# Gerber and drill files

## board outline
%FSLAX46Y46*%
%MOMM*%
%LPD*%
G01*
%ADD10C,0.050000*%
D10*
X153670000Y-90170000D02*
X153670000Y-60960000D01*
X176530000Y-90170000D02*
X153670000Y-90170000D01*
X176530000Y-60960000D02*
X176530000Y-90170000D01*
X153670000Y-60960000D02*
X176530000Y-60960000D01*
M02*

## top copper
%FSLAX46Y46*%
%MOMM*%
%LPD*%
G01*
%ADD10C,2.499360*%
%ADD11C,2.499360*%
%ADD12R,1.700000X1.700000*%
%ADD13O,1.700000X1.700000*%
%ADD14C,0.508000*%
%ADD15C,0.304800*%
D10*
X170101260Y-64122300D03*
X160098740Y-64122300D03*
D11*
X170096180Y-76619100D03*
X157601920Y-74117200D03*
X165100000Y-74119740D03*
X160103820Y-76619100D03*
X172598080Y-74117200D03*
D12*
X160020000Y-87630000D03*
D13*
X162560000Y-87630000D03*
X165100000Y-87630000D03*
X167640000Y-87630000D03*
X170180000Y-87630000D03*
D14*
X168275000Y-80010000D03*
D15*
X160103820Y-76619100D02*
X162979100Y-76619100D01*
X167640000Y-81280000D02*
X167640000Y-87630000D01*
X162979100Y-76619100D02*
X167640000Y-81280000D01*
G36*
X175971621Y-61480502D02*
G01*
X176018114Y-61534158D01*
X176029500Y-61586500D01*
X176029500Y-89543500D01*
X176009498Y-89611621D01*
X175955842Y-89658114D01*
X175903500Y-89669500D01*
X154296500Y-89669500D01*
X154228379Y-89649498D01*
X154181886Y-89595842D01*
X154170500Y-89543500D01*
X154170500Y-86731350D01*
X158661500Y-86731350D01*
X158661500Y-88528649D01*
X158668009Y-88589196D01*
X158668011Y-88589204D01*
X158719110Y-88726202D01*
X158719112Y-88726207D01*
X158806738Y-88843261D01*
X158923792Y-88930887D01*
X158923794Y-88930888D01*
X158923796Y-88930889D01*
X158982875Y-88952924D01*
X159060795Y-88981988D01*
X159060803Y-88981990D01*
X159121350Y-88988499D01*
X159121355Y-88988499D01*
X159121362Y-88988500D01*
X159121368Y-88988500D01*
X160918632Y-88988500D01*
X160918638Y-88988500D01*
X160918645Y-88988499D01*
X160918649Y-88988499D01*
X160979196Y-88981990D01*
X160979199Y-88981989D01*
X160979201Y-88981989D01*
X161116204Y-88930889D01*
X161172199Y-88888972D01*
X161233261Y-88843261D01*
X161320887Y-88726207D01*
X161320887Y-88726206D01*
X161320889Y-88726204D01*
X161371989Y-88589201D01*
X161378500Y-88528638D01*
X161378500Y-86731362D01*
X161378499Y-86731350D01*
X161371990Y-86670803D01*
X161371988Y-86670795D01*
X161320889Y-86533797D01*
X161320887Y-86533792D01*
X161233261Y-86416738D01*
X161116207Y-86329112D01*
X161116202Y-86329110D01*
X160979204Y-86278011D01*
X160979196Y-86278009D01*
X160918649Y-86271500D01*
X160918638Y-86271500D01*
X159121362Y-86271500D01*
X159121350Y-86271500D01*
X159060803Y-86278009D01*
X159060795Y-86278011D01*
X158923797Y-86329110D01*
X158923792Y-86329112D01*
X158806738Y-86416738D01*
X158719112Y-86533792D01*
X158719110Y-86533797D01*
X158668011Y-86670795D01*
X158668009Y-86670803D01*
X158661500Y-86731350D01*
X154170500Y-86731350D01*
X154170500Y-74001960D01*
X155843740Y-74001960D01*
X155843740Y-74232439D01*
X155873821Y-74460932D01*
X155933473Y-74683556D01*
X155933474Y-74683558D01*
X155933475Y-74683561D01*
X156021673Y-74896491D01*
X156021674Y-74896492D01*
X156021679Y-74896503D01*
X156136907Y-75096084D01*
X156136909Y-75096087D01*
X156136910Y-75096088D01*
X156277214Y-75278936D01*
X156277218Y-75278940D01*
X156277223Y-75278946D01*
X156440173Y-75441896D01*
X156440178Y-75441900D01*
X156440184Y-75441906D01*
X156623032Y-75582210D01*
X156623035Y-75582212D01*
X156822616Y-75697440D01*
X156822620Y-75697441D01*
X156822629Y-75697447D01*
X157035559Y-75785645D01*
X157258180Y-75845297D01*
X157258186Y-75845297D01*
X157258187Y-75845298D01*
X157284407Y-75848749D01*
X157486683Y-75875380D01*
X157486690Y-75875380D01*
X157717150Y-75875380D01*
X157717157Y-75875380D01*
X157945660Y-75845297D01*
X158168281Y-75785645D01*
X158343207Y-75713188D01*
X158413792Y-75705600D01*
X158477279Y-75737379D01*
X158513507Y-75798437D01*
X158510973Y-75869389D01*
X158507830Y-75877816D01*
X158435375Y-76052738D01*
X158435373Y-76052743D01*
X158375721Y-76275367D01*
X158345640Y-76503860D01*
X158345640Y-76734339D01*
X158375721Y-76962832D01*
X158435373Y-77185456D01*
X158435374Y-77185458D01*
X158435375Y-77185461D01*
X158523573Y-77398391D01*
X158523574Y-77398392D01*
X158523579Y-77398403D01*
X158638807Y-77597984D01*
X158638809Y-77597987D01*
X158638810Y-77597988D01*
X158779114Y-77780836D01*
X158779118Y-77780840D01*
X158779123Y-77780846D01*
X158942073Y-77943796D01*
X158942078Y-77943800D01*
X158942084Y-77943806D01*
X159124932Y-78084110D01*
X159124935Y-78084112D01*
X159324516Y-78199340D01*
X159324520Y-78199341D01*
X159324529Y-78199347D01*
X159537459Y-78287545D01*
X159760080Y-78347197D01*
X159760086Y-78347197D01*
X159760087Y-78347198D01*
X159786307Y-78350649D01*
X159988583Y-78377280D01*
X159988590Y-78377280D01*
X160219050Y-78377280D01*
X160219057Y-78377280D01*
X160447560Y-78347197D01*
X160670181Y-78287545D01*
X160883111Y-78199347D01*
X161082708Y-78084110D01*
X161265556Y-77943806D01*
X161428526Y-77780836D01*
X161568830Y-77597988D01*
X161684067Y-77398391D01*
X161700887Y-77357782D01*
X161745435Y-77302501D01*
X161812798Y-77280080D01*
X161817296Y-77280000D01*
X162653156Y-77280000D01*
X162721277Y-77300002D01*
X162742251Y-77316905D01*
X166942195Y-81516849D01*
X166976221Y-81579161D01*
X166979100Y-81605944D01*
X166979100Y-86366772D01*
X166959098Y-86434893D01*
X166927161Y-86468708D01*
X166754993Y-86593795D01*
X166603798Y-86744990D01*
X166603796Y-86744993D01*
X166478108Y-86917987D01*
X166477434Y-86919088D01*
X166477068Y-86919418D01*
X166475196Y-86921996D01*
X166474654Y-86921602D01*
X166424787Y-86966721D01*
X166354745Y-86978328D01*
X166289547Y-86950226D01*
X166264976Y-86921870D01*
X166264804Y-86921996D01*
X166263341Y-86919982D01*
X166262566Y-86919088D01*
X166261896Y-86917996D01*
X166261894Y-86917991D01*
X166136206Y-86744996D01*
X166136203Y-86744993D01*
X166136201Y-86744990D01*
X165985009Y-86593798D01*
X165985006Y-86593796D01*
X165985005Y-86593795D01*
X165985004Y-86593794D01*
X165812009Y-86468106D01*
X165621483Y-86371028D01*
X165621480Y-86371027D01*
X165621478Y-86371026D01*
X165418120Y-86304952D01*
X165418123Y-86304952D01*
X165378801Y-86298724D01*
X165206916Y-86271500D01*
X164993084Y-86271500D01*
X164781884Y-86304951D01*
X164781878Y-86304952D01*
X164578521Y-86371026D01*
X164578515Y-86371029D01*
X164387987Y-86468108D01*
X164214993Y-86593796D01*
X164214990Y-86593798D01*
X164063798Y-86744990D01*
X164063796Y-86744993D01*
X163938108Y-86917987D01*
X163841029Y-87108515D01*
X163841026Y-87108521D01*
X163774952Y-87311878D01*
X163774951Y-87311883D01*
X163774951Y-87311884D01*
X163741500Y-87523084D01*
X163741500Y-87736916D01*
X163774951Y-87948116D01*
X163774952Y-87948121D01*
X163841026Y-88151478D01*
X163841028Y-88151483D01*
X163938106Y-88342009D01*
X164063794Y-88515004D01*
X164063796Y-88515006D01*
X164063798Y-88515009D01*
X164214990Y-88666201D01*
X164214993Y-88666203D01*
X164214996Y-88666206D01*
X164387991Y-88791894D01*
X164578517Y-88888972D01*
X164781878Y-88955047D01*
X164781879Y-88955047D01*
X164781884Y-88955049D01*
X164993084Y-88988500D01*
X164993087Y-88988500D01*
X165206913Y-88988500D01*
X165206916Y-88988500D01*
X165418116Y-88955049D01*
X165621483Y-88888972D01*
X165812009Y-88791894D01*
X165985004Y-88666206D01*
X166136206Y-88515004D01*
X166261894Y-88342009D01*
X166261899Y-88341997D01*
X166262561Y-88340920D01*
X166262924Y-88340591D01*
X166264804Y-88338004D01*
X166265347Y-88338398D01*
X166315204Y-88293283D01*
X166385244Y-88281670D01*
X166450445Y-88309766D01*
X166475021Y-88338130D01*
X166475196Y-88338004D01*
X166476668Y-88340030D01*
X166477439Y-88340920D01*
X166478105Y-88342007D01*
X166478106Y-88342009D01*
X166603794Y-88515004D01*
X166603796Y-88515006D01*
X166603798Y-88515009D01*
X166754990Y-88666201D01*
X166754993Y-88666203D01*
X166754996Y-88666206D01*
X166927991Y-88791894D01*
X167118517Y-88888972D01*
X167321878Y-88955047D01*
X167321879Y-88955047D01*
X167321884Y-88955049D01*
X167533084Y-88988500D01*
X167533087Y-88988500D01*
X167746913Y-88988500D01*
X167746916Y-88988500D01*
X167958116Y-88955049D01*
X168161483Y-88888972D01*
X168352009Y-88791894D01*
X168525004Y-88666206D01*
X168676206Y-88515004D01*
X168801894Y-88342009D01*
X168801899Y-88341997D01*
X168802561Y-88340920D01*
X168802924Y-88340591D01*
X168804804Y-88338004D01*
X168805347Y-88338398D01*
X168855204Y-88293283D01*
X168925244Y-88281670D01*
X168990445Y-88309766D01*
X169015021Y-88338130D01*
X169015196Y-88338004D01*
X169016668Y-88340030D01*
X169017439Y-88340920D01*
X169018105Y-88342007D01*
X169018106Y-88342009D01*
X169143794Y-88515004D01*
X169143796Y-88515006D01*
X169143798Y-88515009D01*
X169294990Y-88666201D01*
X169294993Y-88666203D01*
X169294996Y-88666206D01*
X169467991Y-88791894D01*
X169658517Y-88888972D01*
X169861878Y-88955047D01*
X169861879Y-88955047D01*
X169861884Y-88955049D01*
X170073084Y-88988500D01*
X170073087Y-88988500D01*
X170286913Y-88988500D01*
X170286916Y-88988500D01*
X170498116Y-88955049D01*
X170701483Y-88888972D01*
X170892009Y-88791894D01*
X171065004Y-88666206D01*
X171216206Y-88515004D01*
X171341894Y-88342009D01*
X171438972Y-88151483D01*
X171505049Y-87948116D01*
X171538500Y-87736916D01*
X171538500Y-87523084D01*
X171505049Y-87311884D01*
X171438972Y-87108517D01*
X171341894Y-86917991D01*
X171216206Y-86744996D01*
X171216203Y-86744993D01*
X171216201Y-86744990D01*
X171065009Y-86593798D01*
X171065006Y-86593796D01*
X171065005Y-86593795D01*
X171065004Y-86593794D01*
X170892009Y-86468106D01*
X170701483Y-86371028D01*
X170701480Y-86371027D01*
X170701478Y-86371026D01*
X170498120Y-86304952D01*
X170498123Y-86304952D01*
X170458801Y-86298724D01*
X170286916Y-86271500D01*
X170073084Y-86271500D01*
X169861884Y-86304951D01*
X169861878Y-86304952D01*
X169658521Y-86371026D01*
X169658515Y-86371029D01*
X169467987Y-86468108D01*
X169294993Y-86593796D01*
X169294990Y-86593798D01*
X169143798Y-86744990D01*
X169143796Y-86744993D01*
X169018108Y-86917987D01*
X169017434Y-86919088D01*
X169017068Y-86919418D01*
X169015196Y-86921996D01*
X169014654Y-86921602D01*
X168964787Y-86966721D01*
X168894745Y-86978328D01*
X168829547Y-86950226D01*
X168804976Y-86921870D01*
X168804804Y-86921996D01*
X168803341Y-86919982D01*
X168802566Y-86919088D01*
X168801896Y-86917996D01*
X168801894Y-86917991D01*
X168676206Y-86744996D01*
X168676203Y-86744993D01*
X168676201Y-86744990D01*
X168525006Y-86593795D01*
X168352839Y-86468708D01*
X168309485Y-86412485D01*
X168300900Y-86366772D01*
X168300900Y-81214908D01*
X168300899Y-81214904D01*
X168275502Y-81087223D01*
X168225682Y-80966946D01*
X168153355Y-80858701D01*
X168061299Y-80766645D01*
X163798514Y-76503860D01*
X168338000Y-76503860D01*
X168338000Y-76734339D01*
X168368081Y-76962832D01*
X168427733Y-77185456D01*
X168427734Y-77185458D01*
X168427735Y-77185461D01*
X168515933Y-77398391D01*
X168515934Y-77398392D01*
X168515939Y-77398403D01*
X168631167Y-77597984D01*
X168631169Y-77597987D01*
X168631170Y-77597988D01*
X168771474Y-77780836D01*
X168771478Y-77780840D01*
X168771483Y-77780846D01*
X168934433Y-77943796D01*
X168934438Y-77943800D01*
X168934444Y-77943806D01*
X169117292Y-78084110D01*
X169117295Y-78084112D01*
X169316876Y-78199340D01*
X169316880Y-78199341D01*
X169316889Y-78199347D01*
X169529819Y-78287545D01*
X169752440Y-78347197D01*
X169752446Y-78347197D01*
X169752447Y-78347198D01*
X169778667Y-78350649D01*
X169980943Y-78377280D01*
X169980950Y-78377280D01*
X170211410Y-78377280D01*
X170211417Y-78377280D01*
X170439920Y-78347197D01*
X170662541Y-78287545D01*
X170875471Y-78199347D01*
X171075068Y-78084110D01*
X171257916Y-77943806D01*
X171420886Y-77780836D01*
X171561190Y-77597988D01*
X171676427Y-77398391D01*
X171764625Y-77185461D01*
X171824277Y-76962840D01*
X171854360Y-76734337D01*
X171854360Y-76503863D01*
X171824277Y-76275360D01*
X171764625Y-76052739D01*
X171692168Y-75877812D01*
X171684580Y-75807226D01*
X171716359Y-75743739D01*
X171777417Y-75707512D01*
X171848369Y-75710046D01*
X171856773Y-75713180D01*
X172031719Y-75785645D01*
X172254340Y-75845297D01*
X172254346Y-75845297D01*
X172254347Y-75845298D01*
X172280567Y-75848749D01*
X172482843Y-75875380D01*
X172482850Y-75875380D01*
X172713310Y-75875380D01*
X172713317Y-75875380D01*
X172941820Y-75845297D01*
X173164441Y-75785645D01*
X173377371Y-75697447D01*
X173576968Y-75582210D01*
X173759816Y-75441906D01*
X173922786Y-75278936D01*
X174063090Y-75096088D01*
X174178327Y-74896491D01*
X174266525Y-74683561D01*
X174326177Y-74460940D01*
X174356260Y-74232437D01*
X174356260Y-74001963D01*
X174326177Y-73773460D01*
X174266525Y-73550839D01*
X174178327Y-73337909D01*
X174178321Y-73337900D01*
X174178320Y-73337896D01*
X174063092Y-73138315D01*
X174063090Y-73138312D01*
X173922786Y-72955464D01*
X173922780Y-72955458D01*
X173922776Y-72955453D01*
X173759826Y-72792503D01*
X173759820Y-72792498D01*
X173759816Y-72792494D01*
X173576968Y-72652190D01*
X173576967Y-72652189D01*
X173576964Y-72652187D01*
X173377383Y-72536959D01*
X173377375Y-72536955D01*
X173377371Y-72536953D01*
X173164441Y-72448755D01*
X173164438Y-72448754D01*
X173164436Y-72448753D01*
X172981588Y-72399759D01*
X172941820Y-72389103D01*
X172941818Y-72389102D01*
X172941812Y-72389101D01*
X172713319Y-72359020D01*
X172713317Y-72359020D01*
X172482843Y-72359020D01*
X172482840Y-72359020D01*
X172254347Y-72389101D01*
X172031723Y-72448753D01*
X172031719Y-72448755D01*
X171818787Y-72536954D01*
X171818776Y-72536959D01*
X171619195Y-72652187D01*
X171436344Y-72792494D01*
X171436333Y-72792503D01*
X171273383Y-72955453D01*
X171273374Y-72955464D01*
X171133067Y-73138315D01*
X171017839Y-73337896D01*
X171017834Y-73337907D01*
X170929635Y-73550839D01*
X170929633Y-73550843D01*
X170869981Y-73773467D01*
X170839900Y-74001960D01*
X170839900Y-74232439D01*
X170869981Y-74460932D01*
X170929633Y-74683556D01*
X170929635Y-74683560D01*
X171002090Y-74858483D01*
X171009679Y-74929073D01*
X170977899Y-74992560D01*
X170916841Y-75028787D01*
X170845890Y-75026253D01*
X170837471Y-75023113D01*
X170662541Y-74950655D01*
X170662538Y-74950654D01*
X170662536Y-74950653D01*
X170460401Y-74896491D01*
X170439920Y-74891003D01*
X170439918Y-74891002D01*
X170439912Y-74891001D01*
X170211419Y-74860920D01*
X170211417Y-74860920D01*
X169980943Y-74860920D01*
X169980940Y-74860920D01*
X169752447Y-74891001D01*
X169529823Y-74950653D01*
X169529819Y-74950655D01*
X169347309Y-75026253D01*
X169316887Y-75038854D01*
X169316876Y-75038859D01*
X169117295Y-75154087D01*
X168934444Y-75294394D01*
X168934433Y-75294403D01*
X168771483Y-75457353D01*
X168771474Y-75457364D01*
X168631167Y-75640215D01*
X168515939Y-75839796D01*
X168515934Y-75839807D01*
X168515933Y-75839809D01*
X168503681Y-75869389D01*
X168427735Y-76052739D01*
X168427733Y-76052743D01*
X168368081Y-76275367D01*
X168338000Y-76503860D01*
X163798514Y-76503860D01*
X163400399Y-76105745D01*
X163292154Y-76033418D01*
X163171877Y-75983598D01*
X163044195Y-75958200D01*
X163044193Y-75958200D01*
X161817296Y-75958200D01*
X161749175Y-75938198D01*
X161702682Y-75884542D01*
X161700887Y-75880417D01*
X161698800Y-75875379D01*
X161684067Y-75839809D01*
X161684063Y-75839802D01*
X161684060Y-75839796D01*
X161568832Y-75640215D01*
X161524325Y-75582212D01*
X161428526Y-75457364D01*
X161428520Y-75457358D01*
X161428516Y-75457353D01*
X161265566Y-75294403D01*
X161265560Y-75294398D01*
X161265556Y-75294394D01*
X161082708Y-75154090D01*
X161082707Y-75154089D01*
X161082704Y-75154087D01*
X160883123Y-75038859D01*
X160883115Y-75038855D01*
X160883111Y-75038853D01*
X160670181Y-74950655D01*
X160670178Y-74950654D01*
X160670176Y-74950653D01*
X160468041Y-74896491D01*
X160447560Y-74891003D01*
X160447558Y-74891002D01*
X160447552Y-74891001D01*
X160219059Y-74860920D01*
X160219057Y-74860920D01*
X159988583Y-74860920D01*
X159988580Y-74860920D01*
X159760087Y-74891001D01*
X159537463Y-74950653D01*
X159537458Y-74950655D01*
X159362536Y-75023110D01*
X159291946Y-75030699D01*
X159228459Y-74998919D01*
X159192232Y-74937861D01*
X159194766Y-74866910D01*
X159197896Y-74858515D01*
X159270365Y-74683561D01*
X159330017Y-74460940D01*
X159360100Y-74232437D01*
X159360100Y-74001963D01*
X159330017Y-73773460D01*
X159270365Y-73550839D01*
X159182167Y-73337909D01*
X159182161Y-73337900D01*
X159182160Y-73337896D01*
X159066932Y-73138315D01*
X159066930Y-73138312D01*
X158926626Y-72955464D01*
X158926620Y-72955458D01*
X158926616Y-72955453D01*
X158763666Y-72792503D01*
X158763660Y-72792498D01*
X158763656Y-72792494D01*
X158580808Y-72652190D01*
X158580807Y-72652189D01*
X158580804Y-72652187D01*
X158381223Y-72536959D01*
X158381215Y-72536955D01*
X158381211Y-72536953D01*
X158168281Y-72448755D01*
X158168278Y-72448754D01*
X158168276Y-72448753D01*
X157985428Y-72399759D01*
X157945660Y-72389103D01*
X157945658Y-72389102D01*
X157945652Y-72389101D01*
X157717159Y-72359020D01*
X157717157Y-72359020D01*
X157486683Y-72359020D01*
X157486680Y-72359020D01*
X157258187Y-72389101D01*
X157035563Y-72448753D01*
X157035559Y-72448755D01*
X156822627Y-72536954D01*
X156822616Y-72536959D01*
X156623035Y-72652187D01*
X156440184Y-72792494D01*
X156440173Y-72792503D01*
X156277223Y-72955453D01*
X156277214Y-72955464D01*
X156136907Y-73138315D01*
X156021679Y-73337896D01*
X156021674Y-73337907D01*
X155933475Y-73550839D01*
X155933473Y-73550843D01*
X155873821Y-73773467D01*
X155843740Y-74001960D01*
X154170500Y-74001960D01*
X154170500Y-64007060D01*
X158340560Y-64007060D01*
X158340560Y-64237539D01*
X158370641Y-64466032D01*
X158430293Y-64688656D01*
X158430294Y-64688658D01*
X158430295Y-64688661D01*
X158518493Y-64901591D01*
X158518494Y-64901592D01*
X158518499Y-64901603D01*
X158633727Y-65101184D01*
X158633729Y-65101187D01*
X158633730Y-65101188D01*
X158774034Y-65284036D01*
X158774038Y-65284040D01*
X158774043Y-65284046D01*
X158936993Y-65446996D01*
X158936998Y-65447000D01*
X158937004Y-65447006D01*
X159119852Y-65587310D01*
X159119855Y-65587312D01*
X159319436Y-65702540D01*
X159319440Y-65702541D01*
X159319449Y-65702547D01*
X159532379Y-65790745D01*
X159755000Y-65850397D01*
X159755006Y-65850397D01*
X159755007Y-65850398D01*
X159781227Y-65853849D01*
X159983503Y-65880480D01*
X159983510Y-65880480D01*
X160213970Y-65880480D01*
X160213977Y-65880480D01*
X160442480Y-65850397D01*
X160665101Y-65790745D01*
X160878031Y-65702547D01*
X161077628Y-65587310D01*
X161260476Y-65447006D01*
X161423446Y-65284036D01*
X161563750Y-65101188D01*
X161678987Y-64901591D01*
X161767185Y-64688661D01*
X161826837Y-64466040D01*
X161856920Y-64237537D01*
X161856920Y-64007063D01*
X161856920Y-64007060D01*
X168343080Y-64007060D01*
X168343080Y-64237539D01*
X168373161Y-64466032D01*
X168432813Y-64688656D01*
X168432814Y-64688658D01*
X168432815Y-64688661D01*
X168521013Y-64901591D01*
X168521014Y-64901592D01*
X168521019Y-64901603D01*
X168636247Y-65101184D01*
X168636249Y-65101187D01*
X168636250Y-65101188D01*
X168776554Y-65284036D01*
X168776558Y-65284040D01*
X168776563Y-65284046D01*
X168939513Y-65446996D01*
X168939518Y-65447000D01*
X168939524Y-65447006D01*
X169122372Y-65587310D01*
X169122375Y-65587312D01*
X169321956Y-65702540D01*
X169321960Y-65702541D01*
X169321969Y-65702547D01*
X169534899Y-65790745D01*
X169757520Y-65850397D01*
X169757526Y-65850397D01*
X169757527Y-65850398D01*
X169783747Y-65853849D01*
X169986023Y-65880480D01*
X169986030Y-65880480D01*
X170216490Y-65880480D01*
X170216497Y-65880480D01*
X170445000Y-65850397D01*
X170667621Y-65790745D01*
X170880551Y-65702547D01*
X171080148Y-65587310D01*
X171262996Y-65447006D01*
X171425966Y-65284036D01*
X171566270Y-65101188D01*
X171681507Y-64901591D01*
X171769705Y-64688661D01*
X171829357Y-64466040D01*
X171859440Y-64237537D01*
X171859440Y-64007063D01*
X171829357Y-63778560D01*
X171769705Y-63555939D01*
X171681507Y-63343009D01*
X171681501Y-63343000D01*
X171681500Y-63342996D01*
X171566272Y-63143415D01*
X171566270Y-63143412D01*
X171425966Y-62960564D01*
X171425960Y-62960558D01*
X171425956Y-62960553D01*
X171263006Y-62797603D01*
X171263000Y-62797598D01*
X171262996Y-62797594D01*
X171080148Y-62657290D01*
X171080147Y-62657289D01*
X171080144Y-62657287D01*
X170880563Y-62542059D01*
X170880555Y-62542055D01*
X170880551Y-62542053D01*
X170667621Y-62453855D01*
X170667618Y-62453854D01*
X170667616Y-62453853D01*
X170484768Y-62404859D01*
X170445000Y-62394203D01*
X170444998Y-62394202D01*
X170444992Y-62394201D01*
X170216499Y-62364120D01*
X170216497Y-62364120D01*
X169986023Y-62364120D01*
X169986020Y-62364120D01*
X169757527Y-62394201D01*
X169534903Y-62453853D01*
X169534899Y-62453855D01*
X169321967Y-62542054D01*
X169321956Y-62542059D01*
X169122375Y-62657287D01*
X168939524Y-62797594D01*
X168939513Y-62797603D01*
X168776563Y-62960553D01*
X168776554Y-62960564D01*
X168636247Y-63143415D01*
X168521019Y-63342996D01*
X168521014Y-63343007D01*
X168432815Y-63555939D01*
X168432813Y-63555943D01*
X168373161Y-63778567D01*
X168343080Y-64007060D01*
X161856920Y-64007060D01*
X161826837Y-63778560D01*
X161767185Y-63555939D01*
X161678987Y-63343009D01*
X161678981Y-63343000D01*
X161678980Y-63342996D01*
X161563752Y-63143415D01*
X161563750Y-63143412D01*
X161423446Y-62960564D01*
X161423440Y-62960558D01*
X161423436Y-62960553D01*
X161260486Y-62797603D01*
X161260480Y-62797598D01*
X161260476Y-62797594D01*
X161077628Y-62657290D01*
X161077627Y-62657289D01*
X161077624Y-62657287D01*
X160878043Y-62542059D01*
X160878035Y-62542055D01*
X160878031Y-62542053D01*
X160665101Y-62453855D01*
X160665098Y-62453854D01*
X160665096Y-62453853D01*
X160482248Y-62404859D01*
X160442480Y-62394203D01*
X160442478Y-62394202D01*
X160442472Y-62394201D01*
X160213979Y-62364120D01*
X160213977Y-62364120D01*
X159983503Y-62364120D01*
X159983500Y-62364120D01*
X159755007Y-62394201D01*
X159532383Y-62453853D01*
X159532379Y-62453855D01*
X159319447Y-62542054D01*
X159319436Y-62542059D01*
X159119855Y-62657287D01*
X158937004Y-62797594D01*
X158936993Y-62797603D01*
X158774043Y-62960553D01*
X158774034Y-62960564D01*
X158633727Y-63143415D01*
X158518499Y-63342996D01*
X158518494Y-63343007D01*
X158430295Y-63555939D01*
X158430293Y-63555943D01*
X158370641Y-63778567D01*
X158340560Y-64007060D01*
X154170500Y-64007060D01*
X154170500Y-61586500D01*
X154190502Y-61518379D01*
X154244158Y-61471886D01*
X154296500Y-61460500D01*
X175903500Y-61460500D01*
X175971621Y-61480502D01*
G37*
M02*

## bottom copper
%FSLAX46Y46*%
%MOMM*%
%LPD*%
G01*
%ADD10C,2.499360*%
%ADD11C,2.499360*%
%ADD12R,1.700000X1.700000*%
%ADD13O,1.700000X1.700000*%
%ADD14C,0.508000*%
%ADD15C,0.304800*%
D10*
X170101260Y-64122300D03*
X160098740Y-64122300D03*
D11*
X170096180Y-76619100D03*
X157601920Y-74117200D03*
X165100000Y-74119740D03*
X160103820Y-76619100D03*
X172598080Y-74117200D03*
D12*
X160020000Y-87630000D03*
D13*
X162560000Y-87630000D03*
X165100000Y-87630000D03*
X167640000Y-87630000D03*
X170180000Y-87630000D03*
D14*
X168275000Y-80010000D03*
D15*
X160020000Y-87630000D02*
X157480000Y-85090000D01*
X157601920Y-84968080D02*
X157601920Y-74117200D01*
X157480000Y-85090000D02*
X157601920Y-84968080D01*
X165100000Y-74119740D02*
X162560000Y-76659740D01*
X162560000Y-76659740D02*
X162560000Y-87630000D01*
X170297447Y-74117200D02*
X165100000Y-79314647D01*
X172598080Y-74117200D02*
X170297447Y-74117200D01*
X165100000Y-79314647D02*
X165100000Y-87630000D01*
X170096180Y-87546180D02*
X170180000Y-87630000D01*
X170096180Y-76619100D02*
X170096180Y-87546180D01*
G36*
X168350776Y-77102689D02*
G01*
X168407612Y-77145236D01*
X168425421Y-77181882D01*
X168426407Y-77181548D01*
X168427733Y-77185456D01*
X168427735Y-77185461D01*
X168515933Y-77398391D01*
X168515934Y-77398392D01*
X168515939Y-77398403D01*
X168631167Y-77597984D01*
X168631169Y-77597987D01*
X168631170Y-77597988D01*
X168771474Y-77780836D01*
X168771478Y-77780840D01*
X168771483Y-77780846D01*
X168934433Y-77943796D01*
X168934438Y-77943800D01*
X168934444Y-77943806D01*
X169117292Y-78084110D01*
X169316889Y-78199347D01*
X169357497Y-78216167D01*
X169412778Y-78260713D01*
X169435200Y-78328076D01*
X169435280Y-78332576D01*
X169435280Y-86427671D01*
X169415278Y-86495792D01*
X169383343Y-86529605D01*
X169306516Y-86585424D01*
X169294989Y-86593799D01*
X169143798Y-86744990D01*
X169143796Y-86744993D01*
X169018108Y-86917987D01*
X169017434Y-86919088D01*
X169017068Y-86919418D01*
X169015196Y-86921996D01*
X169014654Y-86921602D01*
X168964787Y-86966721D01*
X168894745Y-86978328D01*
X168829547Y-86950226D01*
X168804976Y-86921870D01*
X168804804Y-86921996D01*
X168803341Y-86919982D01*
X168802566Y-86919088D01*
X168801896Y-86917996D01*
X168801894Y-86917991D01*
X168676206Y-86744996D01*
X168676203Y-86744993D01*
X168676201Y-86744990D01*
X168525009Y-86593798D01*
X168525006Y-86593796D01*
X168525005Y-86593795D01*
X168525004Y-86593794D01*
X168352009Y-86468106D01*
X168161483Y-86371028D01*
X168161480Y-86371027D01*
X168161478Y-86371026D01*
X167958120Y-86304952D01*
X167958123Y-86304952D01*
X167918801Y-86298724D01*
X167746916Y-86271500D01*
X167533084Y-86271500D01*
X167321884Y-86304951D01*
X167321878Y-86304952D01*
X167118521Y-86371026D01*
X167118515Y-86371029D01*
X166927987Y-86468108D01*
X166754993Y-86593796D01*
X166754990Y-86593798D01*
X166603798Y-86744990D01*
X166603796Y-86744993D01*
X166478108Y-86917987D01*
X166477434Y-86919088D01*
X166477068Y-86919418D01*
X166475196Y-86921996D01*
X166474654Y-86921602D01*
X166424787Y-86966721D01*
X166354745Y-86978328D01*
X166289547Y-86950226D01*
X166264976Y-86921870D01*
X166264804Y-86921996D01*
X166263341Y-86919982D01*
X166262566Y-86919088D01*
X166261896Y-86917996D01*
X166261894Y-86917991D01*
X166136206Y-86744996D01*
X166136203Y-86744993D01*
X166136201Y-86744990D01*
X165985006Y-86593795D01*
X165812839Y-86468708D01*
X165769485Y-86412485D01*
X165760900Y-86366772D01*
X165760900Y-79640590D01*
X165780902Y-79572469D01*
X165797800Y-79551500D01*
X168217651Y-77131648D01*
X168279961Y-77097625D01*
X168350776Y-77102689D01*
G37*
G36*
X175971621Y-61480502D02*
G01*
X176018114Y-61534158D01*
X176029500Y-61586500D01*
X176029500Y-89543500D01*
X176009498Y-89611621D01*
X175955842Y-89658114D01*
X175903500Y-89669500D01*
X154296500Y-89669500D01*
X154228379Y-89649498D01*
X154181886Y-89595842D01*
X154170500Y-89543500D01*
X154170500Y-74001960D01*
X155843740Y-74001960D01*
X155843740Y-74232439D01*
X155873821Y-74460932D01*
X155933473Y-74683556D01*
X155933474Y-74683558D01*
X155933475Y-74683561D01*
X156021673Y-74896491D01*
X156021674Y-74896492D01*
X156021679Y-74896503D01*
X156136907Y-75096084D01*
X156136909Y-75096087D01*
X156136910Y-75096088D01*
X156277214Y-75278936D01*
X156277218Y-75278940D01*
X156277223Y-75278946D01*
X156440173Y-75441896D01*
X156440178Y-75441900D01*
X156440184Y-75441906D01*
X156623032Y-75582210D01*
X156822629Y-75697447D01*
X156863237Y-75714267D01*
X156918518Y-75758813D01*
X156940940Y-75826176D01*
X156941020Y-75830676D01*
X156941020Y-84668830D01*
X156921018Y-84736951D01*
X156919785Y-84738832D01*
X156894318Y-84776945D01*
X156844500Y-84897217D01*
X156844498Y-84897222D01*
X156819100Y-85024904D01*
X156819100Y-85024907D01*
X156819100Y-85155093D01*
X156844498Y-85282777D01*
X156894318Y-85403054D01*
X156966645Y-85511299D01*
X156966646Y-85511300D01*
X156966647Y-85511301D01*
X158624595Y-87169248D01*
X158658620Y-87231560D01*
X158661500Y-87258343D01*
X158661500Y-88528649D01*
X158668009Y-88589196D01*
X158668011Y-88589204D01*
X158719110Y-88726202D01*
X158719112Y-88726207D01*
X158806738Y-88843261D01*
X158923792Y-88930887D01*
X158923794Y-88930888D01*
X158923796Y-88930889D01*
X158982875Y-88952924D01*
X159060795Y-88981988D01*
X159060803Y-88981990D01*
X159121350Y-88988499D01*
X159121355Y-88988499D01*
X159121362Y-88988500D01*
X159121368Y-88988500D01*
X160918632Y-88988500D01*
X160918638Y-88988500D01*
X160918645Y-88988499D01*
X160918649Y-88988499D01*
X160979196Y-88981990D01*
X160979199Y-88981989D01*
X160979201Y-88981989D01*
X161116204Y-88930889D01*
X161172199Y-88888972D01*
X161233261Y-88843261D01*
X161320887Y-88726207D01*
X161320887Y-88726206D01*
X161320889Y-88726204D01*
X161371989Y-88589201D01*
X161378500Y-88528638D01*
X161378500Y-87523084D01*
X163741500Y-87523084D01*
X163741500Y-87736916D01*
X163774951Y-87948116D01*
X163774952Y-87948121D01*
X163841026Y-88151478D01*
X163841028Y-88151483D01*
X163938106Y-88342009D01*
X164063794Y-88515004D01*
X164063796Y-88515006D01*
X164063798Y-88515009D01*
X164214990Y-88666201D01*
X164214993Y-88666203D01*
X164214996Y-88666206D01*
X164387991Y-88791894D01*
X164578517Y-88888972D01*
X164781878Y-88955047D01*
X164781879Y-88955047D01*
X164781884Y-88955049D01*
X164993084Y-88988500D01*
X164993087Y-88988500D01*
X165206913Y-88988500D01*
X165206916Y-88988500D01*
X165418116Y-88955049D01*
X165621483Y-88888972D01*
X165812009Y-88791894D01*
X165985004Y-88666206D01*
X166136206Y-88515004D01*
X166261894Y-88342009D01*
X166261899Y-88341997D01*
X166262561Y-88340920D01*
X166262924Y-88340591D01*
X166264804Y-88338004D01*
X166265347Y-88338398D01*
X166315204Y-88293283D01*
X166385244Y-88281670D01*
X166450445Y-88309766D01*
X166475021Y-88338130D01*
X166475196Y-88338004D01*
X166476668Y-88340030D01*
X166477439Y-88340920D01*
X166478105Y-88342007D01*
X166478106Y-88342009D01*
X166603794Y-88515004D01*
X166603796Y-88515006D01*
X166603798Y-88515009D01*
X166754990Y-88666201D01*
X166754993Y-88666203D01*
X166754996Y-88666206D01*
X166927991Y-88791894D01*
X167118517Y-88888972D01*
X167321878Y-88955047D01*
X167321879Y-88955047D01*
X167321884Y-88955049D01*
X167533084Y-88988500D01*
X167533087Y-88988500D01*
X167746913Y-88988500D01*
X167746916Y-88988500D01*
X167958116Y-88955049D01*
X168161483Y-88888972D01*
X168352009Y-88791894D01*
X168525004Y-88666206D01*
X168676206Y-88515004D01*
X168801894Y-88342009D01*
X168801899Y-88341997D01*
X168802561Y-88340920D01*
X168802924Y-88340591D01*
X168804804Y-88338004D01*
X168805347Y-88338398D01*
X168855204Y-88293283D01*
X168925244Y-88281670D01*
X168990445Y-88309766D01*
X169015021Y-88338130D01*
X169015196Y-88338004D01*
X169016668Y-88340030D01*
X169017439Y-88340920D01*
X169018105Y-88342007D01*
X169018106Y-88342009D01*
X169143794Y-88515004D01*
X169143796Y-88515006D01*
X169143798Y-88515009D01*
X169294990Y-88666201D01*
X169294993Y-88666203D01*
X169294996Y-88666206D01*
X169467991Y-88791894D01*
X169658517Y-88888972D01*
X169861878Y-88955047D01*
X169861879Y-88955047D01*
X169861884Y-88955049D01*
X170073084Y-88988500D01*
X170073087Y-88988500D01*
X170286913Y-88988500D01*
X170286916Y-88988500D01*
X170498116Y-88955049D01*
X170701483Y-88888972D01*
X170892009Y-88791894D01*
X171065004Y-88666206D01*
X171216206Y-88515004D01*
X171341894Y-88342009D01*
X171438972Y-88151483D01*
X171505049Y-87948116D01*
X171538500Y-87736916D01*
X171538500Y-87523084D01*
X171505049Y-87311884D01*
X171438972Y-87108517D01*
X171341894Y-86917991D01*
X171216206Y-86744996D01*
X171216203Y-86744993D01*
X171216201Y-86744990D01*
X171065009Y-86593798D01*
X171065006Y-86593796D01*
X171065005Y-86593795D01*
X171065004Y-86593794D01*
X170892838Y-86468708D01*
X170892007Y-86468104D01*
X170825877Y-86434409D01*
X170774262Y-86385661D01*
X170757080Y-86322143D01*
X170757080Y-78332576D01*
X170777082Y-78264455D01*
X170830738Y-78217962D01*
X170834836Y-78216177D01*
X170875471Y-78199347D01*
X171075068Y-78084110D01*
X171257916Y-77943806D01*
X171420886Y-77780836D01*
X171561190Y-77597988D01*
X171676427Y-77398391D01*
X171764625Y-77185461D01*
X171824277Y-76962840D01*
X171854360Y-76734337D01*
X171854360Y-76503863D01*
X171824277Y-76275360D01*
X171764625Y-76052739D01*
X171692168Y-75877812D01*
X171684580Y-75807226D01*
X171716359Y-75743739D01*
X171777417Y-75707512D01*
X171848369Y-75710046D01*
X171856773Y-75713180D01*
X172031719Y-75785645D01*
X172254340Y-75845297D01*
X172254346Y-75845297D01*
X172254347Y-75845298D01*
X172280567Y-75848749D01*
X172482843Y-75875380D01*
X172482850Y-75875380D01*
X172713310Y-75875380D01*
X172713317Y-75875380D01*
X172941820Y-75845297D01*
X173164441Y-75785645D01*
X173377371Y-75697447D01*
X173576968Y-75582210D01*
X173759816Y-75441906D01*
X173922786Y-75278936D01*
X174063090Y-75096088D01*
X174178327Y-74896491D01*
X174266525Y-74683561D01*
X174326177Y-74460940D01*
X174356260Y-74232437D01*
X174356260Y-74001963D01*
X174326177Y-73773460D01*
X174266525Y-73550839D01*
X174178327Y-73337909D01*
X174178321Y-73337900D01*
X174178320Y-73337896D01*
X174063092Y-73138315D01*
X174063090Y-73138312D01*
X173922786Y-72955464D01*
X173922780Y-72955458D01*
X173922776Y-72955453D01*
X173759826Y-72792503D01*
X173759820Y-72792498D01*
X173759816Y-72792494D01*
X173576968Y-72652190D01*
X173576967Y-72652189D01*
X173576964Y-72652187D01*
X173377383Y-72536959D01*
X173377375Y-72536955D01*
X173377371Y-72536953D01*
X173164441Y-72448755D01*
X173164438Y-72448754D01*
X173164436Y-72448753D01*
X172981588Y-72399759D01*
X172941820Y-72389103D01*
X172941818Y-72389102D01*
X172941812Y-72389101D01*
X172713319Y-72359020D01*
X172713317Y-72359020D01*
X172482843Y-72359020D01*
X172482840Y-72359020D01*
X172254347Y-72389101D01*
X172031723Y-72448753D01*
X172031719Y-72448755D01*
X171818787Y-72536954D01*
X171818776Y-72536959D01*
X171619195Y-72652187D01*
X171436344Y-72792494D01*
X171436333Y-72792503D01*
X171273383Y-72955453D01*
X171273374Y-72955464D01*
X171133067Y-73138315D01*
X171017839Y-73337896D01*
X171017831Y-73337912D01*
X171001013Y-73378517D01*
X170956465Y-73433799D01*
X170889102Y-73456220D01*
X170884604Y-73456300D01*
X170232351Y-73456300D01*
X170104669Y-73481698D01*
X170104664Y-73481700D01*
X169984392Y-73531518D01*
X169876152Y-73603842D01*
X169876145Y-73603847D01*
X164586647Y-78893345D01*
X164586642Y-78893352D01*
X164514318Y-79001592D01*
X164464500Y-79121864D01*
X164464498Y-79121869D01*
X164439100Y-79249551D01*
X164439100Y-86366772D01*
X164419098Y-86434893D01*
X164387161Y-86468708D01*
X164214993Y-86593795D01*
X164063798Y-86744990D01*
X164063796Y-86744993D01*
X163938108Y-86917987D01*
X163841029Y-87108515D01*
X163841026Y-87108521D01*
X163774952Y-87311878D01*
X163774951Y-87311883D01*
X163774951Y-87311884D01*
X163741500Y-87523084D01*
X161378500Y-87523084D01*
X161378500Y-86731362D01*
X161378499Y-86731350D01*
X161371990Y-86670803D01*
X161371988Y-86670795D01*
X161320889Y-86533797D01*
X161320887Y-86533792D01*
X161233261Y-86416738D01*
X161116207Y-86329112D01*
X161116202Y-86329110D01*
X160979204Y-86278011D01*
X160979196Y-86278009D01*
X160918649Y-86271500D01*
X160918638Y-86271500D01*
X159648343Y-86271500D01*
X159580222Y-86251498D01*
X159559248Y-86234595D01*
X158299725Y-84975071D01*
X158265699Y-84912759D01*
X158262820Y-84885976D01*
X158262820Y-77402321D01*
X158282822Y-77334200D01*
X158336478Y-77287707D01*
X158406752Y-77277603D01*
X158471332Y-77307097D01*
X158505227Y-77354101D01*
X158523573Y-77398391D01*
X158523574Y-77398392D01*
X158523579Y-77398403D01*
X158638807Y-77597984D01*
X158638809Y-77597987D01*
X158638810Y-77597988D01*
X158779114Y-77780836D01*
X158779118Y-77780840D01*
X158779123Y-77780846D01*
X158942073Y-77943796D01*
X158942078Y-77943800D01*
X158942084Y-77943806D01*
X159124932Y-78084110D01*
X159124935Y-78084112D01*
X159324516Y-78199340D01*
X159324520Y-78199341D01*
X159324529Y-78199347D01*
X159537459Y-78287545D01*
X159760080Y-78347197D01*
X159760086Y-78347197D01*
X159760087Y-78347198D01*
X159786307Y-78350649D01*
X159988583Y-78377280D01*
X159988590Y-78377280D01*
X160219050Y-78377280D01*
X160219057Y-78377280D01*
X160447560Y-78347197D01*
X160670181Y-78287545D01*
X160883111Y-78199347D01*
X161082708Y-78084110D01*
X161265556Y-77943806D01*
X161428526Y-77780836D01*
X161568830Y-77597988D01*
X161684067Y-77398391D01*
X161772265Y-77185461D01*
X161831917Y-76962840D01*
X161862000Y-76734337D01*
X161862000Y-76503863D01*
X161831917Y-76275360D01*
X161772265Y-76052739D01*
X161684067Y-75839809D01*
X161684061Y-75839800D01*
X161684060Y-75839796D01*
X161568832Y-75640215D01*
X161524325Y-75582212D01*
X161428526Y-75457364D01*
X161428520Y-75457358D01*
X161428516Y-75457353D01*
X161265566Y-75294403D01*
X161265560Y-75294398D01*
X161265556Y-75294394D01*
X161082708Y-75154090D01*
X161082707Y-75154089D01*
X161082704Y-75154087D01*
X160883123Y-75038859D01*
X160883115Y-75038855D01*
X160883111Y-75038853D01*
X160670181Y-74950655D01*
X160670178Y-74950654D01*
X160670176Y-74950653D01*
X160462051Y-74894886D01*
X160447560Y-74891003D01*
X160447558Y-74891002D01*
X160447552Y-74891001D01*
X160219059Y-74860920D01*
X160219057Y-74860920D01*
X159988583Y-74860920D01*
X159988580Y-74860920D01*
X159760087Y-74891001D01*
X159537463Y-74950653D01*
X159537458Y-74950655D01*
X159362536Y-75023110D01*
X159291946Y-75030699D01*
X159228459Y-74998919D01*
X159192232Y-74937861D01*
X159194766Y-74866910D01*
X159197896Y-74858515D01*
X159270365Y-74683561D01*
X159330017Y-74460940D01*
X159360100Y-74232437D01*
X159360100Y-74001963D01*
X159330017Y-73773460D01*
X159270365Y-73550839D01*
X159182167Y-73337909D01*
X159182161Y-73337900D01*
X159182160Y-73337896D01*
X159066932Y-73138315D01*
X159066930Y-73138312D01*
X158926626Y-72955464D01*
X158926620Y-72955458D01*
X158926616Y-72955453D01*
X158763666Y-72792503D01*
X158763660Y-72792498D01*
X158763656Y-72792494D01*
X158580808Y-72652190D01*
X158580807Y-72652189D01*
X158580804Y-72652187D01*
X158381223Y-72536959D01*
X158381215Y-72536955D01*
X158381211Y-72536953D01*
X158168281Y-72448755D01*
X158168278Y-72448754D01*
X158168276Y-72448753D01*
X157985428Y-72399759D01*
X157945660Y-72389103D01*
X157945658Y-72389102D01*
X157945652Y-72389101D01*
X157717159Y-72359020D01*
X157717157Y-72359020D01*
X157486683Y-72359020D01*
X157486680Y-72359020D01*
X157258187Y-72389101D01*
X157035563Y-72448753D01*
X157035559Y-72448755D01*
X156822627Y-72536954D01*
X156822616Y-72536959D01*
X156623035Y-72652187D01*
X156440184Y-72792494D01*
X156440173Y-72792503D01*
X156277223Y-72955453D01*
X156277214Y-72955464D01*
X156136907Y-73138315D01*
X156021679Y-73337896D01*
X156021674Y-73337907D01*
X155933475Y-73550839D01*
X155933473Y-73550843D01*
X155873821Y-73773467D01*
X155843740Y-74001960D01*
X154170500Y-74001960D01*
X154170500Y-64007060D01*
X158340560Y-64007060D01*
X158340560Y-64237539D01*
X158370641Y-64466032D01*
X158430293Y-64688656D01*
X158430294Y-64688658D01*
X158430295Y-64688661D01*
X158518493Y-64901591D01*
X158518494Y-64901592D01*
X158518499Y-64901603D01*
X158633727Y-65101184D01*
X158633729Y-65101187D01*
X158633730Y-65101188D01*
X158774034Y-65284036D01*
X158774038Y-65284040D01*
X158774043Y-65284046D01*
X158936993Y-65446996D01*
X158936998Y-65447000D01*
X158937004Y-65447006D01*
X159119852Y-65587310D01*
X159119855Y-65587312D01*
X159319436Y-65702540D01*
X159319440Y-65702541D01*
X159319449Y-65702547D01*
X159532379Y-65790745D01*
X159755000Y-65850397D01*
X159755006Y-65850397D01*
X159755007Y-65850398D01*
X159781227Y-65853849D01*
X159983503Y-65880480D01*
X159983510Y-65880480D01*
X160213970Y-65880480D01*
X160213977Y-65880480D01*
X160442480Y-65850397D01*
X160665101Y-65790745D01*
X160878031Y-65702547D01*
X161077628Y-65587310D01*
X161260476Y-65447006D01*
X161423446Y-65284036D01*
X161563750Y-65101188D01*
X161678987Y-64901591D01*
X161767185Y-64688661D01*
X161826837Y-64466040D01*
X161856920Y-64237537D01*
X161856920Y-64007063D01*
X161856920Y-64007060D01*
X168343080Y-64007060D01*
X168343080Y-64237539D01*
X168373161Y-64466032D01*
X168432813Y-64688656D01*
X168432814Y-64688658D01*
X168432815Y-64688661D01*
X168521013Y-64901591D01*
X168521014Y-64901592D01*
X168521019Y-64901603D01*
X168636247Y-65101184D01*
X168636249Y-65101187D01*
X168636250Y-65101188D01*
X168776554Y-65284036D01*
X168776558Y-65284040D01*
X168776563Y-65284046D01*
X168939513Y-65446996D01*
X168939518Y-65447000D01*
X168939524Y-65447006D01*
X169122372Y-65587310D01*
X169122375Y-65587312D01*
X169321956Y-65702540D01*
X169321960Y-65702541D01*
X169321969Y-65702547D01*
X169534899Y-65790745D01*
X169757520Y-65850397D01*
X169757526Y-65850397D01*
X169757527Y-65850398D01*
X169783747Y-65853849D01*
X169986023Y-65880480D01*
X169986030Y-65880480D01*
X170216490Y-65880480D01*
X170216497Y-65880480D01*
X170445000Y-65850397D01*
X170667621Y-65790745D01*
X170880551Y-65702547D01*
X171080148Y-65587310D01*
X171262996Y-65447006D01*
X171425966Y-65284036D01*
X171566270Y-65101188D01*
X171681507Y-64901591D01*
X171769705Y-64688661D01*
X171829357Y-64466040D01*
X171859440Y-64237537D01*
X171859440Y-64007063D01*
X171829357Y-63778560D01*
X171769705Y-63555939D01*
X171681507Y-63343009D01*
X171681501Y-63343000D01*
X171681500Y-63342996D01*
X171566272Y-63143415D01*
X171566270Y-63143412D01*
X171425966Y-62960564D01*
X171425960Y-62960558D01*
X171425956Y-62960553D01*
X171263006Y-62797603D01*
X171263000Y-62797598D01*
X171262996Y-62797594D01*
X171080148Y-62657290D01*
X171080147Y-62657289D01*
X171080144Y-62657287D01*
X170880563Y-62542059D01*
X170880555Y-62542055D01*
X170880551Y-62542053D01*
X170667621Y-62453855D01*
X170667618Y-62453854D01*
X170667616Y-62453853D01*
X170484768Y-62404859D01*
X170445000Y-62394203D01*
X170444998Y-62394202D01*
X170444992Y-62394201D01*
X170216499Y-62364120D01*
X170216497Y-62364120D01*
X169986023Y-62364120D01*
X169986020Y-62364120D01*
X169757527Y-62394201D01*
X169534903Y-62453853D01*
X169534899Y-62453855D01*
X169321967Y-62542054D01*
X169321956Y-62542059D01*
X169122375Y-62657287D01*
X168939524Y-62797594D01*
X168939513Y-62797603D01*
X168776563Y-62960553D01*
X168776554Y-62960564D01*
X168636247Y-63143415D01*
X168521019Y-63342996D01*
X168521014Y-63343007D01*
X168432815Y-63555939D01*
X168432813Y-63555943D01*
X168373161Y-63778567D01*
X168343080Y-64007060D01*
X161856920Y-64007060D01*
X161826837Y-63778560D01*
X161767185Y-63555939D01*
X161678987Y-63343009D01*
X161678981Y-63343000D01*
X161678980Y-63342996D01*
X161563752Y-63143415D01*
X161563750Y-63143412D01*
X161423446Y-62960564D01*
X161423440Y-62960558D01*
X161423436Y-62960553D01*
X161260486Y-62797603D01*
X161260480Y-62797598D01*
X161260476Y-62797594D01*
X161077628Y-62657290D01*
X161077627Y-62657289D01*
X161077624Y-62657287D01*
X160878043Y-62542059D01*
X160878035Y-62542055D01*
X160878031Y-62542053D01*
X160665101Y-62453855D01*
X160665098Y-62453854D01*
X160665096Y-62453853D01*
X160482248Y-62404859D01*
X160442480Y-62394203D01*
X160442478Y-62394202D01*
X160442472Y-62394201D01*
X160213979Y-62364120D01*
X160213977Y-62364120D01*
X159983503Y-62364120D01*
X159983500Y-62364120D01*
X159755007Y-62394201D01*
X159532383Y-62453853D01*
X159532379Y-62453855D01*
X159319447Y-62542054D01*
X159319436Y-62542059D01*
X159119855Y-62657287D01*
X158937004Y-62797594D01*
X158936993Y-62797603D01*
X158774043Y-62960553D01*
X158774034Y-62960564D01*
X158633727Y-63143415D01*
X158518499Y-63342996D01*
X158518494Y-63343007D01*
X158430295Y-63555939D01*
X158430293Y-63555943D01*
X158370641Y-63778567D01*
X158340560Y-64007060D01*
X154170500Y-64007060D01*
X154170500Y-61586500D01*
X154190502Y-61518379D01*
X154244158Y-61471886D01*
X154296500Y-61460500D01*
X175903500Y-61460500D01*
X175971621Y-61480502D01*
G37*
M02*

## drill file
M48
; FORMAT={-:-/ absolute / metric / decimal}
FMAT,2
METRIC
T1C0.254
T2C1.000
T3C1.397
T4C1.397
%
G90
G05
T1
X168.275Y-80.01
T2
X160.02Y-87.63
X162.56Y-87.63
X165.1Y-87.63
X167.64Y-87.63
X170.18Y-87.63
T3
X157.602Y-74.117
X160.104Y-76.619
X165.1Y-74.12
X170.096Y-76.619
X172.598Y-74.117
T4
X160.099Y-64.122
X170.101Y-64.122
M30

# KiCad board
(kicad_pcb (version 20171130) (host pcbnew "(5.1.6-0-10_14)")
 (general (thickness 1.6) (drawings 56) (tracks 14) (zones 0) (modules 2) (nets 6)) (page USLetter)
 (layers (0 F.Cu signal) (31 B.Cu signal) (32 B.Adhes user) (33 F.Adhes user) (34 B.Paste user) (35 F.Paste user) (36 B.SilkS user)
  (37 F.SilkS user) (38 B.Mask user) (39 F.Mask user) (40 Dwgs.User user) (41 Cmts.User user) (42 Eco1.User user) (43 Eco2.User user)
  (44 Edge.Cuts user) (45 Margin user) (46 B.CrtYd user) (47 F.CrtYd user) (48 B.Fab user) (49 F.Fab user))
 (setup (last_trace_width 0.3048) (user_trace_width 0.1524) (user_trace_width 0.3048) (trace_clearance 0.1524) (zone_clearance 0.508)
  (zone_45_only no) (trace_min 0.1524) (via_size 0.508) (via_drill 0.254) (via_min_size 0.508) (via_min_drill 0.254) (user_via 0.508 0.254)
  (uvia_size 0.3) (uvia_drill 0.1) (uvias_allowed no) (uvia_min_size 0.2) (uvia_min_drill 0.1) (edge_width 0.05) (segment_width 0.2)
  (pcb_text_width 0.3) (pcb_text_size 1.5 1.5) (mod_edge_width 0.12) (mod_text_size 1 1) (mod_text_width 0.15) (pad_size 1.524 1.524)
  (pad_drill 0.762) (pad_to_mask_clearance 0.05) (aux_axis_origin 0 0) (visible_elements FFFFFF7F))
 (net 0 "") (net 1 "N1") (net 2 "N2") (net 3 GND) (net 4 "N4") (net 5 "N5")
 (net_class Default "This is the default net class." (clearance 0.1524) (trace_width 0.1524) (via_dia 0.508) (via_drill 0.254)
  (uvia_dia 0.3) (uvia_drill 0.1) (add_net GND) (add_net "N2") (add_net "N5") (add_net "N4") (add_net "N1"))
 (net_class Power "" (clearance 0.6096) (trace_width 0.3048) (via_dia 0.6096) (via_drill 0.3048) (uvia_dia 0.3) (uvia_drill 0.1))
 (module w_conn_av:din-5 (layer F.Cu) (at 165.1 71.12 180)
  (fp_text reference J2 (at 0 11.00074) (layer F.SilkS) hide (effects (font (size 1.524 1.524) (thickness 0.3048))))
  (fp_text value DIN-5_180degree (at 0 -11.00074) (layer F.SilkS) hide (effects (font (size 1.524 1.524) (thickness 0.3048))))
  (pad "" np_thru_hole circle (at -5.00126 6.9977 180) (size 2.49936 2.49936) (drill 1.397) (layers *.Cu *.Mask F.SilkS))
  (pad "" np_thru_hole circle (at 5.00126 6.9977 180) (size 2.49936 2.49936) (drill 1.397) (layers *.Cu *.Mask F.SilkS))
  (pad 5 thru_hole circle (at -4.99618 -5.4991 180) (size 2.49936 2.49936) (drill 1.397) (layers *.Cu *.SilkS *.Mask) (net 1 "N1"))
  (pad 1 thru_hole circle (at 7.49808 -2.9972 180) (size 2.49936 2.49936) (drill 1.397) (layers *.Cu *.SilkS *.Mask) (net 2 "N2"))
  (pad 2 thru_hole circle (at 0 -2.99974 180) (size 2.49936 2.49936) (drill 1.397) (layers *.Cu *.SilkS *.Mask) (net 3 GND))
  (pad 4 thru_hole circle (at 4.99618 -5.4991 180) (size 2.49936 2.49936) (drill 1.397) (layers *.Cu *.SilkS *.Mask) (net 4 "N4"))
  (pad 3 thru_hole circle (at -7.49808 -2.9972 180) (size 2.49936 2.49936) (drill 1.397) (layers *.Cu *.SilkS *.Mask) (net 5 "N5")))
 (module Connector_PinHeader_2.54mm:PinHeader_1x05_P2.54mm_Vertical (layer F.Cu) (at 160.02 87.63 90)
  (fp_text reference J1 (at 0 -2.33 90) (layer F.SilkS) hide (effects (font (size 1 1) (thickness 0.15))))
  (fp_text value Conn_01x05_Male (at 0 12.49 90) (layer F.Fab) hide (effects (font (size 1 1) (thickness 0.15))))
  (pad 1 thru_hole rect (at 0 0 90) (size 1.7 1.7) (drill 1) (layers *.Cu *.Mask) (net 2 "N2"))
  (pad 2 thru_hole oval (at 0 2.54 90) (size 1.7 1.7) (drill 1) (layers *.Cu *.Mask) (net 3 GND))
  (pad 3 thru_hole oval (at 0 5.08 90) (size 1.7 1.7) (drill 1) (layers *.Cu *.Mask) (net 5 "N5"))
  (pad 4 thru_hole oval (at 0 7.62 90) (size 1.7 1.7) (drill 1) (layers *.Cu *.Mask) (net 4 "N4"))
  (pad 5 thru_hole oval (at 0 10.16 90) (size 1.7 1.7) (drill 1) (layers *.Cu *.Mask) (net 1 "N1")))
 (gr_line (start 153.67 90.17) (end 153.67 60.96) (layer Edge.Cuts) (width 0.05))
 (gr_line (start 176.53 90.17) (end 153.67 90.17) (layer Edge.Cuts) (width 0.05))
 (gr_line (start 176.53 60.96) (end 176.53 90.17) (layer Edge.Cuts) (width 0.05))
 (gr_line (start 153.67 60.96) (end 176.53 60.96) (layer Edge.Cuts) (width 0.05))
 (segment (start 160.02 87.63) (end 157.48 85.09) (width 0.3048) (layer B.Cu) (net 2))
 (segment (start 157.60192 84.96808) (end 157.60192 74.1172) (width 0.3048) (layer B.Cu) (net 2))
 (segment (start 157.48 85.09) (end 157.60192 84.96808) (width 0.3048) (layer B.Cu) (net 2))
 (segment (start 165.1 74.11974) (end 162.56 76.65974) (width 0.3048) (layer B.Cu) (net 3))
 (segment (start 162.56 76.65974) (end 162.56 87.63) (width 0.3048) (layer B.Cu) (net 3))
 (via (at 168.275 80.01) (size 0.508) (drill 0.254) (layers F.Cu B.Cu) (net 3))
 (segment (start 170.297447 74.1172) (end 165.1 79.314647) (width 0.3048) (layer B.Cu) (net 5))
 (segment (start 172.59808 74.1172) (end 170.297447 74.1172) (width 0.3048) (layer B.Cu) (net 5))
 (segment (start 165.1 79.314647) (end 165.1 87.63) (width 0.3048) (layer B.Cu) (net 5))
 (segment (start 160.10382 76.6191) (end 162.9791 76.6191) (width 0.3048) (layer F.Cu) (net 4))
 (segment (start 167.64 81.28) (end 167.64 87.63) (width 0.3048) (layer F.Cu) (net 4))
 (segment (start 162.9791 76.6191) (end 167.64 81.28) (width 0.3048) (layer F.Cu) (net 4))
 (segment (start 170.09618 87.54618) (end 170.18 87.63) (width 0.3048) (layer B.Cu) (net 1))
 (segment (start 170.09618 76.6191) (end 170.09618 87.54618) (width 0.3048) (layer B.Cu) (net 1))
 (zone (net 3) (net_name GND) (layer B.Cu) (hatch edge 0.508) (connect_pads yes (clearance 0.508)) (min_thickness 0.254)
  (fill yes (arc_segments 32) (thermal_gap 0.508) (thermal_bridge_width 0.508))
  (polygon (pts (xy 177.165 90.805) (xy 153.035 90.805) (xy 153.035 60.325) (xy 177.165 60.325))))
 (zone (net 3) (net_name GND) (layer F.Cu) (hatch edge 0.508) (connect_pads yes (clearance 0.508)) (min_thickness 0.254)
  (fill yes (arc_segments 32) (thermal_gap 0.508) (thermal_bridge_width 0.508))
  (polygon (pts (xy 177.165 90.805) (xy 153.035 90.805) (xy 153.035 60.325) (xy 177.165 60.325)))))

